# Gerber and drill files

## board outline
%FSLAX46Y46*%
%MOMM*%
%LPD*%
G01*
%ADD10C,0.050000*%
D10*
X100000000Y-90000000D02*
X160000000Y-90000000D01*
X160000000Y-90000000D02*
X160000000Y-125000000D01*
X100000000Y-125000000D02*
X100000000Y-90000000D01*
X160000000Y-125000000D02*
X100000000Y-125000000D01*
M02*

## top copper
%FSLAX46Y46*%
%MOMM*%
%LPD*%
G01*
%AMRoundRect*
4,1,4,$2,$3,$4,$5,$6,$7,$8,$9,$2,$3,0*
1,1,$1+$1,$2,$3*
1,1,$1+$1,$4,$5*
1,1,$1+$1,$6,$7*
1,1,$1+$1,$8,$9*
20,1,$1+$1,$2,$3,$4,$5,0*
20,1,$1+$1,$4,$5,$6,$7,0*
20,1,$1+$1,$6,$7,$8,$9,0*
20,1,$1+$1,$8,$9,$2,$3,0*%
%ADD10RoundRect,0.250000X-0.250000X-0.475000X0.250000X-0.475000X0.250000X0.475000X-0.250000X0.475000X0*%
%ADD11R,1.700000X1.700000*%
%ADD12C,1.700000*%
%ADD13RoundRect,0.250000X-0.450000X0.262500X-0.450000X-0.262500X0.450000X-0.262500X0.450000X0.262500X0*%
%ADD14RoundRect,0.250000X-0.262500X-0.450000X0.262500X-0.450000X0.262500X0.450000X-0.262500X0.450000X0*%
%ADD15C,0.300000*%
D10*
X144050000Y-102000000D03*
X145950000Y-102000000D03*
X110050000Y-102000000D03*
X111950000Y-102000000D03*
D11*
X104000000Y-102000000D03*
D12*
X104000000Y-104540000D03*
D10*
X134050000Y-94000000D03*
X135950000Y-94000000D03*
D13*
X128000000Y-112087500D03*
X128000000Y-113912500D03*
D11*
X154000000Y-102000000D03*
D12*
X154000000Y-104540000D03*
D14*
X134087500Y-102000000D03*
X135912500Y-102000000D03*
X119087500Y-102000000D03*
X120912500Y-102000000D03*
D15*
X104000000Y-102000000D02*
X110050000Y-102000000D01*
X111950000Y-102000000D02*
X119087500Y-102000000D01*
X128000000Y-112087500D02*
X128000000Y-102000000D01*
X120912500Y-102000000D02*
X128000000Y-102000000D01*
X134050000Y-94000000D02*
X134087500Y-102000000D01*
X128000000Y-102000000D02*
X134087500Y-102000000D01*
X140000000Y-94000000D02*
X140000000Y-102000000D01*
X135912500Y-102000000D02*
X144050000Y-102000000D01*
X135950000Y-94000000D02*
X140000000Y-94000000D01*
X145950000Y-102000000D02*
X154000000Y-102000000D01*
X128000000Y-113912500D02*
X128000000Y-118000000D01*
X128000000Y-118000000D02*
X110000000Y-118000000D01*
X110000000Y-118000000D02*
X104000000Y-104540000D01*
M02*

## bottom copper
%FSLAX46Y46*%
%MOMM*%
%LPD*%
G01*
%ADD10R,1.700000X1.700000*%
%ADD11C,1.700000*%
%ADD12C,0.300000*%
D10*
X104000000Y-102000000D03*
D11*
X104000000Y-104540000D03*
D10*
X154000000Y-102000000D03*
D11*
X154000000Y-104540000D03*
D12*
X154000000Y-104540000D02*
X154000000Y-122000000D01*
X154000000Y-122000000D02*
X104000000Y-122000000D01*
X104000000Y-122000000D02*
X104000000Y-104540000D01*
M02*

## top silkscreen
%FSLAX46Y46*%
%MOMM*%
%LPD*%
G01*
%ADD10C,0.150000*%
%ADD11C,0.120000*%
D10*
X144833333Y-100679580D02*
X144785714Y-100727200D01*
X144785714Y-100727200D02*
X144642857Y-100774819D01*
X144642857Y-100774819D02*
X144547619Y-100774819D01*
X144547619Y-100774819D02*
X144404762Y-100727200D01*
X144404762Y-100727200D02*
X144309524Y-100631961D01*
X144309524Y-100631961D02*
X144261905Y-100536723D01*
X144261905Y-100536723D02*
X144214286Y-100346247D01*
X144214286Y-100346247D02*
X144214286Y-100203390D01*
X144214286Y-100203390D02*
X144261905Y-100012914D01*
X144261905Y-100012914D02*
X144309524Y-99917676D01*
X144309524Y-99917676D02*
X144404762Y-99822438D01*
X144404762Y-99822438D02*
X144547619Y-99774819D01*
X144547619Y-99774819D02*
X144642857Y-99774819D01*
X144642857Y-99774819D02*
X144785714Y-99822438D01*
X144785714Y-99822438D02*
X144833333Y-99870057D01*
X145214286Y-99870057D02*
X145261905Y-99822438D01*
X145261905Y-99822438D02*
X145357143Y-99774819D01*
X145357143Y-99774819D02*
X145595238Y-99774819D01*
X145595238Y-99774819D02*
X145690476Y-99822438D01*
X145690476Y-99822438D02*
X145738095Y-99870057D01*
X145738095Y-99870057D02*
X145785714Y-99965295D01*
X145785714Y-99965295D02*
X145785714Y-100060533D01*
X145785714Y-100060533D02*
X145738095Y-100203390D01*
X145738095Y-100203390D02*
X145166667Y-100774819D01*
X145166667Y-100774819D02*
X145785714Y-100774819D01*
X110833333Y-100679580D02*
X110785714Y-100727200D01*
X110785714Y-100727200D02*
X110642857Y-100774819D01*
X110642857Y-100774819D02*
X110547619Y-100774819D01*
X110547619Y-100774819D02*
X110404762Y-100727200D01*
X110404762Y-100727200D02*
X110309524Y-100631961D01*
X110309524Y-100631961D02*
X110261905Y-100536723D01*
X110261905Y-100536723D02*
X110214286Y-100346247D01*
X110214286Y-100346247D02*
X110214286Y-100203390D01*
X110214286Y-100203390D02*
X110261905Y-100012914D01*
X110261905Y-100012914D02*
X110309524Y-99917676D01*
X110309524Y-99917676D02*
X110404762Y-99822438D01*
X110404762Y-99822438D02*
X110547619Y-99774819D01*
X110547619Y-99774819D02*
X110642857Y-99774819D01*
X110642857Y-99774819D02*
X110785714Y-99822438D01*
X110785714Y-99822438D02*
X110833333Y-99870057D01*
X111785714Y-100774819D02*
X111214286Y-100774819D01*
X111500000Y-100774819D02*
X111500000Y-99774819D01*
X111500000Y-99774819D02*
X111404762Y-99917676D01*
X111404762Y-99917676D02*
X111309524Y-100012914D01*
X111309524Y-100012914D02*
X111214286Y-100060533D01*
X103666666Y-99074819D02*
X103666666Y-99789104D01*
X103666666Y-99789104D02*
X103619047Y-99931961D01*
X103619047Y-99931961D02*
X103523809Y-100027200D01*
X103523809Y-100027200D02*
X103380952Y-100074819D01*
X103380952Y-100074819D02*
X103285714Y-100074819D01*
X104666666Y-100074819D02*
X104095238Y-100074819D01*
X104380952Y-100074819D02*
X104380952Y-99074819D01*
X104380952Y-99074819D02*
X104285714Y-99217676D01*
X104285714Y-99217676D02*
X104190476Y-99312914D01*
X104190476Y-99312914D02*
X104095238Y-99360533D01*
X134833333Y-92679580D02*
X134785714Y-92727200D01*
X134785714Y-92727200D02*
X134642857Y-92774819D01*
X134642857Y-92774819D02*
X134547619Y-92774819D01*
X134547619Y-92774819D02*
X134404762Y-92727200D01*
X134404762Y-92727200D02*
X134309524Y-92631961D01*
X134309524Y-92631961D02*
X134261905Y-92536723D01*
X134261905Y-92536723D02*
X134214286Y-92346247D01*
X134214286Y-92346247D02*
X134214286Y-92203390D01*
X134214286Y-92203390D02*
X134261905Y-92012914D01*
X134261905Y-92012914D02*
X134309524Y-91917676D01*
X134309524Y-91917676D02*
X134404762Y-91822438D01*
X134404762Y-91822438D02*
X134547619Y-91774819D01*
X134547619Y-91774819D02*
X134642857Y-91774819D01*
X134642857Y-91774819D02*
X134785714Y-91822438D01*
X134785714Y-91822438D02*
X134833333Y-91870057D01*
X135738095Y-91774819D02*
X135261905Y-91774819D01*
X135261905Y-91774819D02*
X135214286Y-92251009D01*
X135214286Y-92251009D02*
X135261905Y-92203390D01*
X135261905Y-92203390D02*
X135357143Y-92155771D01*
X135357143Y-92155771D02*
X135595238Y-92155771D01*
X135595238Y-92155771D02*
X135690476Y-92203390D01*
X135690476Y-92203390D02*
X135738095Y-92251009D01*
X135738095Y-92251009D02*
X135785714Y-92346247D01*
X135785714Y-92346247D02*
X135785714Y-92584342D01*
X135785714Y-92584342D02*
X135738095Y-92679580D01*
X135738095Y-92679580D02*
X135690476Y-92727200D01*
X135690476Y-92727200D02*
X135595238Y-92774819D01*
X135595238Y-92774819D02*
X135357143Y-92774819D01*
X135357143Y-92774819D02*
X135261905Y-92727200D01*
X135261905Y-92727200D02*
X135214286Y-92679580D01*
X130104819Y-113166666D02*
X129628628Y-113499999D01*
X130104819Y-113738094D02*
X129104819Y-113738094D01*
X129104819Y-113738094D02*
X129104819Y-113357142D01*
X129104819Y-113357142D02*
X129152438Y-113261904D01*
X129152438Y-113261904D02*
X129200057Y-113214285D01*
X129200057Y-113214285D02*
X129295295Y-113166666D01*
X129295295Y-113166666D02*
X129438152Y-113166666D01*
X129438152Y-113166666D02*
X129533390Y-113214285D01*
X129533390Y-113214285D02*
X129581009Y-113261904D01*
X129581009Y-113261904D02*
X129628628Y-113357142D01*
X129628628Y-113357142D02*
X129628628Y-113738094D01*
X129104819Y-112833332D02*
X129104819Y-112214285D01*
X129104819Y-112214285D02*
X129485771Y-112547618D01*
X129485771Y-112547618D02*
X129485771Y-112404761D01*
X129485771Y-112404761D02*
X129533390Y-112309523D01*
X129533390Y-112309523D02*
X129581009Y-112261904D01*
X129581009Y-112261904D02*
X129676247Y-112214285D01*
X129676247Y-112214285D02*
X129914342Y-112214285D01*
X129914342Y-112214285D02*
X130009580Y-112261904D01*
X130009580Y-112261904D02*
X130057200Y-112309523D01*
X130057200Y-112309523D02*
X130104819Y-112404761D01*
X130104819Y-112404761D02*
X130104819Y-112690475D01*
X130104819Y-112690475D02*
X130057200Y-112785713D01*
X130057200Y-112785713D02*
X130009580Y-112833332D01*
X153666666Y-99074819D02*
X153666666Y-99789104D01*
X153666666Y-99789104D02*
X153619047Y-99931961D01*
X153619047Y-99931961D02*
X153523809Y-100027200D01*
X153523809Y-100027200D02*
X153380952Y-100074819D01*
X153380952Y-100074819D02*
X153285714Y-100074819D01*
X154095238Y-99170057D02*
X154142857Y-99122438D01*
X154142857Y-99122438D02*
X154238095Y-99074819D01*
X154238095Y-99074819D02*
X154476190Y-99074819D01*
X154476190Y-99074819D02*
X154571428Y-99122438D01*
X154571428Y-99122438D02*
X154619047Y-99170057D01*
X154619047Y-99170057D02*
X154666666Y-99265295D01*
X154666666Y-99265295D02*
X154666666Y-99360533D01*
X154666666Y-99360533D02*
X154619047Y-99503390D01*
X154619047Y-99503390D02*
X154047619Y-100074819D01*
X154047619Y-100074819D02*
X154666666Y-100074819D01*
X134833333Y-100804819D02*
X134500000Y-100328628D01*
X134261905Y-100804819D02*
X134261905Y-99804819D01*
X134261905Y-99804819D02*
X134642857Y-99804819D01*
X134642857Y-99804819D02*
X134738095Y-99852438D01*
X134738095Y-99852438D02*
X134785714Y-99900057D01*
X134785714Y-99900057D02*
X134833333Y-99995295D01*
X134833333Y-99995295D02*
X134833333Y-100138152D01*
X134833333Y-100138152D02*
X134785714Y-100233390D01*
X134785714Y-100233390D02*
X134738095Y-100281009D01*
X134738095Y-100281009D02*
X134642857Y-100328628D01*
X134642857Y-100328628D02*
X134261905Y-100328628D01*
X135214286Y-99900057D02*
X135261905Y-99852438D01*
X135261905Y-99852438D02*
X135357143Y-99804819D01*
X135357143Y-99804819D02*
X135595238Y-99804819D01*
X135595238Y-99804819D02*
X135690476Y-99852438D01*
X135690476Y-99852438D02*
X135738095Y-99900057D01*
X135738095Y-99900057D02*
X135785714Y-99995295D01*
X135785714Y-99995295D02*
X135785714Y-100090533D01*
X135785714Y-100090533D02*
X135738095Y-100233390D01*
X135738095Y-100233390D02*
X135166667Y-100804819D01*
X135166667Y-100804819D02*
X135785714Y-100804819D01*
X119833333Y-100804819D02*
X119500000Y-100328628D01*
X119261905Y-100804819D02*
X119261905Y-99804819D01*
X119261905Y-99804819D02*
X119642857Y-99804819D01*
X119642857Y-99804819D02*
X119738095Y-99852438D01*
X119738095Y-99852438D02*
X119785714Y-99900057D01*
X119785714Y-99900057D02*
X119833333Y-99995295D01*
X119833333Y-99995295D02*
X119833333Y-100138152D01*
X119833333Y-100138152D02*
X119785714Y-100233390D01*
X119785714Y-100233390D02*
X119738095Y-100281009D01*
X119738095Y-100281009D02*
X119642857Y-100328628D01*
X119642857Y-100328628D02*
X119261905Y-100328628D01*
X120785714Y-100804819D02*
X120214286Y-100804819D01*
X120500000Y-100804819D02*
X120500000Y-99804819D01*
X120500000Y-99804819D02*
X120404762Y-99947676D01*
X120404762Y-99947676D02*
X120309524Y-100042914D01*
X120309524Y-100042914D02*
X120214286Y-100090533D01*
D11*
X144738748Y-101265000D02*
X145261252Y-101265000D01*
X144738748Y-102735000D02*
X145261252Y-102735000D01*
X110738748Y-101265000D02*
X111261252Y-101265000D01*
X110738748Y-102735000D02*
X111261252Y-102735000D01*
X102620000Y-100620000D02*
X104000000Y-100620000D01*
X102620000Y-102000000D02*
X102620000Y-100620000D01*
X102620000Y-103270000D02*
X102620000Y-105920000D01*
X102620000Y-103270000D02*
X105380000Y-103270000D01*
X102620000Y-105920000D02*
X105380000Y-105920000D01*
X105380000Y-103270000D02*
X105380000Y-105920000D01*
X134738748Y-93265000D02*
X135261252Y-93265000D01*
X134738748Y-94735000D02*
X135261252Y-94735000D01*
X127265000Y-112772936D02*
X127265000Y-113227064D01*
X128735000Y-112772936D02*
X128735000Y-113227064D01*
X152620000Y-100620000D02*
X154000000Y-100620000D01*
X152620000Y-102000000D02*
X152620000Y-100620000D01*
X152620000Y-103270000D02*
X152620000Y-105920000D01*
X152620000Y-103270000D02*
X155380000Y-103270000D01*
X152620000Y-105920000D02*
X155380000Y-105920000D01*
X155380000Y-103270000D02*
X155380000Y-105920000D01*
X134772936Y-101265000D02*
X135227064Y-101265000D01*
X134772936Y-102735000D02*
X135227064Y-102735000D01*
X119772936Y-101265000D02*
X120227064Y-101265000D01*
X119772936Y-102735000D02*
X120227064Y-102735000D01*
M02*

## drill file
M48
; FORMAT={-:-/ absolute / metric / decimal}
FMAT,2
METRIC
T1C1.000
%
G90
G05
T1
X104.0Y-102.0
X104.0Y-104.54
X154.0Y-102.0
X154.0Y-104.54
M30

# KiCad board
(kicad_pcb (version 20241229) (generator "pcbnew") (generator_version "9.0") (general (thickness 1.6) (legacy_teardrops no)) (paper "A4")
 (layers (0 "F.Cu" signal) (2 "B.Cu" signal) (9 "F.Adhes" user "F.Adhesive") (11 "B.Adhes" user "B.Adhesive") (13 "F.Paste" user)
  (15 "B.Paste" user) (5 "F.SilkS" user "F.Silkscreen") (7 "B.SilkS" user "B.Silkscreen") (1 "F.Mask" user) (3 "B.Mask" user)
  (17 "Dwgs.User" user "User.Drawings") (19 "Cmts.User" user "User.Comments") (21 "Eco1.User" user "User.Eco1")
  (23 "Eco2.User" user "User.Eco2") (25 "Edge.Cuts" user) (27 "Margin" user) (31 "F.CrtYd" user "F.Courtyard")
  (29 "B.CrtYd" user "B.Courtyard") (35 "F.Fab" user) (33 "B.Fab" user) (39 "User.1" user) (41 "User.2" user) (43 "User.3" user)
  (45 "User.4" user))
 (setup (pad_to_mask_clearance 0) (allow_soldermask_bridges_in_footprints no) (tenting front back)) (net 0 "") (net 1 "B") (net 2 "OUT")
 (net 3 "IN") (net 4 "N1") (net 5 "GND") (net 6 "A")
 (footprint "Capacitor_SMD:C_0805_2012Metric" (layer "F.Cu") (at 145 102)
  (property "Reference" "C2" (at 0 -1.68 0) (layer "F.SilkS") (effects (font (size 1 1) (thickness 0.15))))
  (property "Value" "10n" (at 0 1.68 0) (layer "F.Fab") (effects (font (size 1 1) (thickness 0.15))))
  (fp_line (start -0.261252 -0.735) (end 0.261252 -0.735) (stroke (width 0.12) (type solid)) (layer "F.SilkS"))
  (fp_line (start -0.261252 0.735) (end 0.261252 0.735) (stroke (width 0.12) (type solid)) (layer "F.SilkS"))
  (pad "1" smd roundrect (at -0.95 0) (size 1 1.45) (layers "F.Cu" "F.Mask" "F.Paste") (roundrect_rratio 0.25) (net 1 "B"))
  (pad "2" smd roundrect (at 0.95 0) (size 1 1.45) (layers "F.Cu" "F.Mask" "F.Paste") (roundrect_rratio 0.25) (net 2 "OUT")))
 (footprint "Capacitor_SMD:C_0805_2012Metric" (layer "F.Cu") (at 111 102)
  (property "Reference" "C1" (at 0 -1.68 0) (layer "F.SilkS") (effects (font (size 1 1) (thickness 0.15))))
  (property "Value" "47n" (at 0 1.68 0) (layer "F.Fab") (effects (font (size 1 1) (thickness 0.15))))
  (fp_line (start -0.261252 -0.735) (end 0.261252 -0.735) (stroke (width 0.12) (type solid)) (layer "F.SilkS"))
  (fp_line (start -0.261252 0.735) (end 0.261252 0.735) (stroke (width 0.12) (type solid)) (layer "F.SilkS"))
  (pad "1" smd roundrect (at -0.95 0) (size 1 1.45) (layers "F.Cu" "F.Mask" "F.Paste") (roundrect_rratio 0.25) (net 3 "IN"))
  (pad "2" smd roundrect (at 0.95 0) (size 1 1.45) (layers "F.Cu" "F.Mask" "F.Paste") (roundrect_rratio 0.25) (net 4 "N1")))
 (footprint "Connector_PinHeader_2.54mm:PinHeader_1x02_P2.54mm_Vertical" (layer "F.Cu") (at 104 102)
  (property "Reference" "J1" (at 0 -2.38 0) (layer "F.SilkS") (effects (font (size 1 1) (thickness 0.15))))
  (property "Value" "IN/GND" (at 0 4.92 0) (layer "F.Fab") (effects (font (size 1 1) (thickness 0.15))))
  (fp_line (start -1.38 -1.38) (end 0 -1.38) (stroke (width 0.12) (type solid)) (layer "F.SilkS"))
  (fp_line (start -1.38 0) (end -1.38 -1.38) (stroke (width 0.12) (type solid)) (layer "F.SilkS"))
  (fp_line (start -1.38 1.27) (end -1.38 3.92) (stroke (width 0.12) (type solid)) (layer "F.SilkS"))
  (fp_line (start -1.38 1.27) (end 1.38 1.27) (stroke (width 0.12) (type solid)) (layer "F.SilkS"))
  (fp_line (start -1.38 3.92) (end 1.38 3.92) (stroke (width 0.12) (type solid)) (layer "F.SilkS"))
  (fp_line (start 1.38 1.27) (end 1.38 3.92) (stroke (width 0.12) (type solid)) (layer "F.SilkS"))
  (pad "1" thru_hole rect (at 0 0) (size 1.7 1.7) (drill 1) (layers "*.Cu" "*.Mask") (remove_unused_layers no) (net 3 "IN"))
  (pad "2" thru_hole circle (at 0 2.54) (size 1.7 1.7) (drill 1) (layers "*.Cu" "*.Mask") (remove_unused_layers no) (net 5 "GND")))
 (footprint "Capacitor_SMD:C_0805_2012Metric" (layer "F.Cu") (at 135 94)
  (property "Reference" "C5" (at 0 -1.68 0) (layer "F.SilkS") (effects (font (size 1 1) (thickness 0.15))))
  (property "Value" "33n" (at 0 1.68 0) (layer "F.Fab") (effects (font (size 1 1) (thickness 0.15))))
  (fp_line (start -0.261252 -0.735) (end 0.261252 -0.735) (stroke (width 0.12) (type solid)) (layer "F.SilkS"))
  (fp_line (start -0.261252 0.735) (end 0.261252 0.735) (stroke (width 0.12) (type solid)) (layer "F.SilkS"))
  (pad "1" smd roundrect (at -0.95 0) (size 1 1.45) (layers "F.Cu" "F.Mask" "F.Paste") (roundrect_rratio 0.25) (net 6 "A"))
  (pad "2" smd roundrect (at 0.95 0) (size 1 1.45) (layers "F.Cu" "F.Mask" "F.Paste") (roundrect_rratio 0.25) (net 1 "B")))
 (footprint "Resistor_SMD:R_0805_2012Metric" (layer "F.Cu") (at 128 113 -90)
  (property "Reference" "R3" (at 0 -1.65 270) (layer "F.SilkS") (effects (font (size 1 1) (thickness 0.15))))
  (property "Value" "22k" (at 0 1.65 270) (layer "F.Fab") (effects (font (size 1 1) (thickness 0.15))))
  (fp_line (start -0.227064 0.735) (end 0.227064 0.735) (stroke (width 0.12) (type solid)) (layer "F.SilkS"))
  (fp_line (start -0.227064 -0.735) (end 0.227064 -0.735) (stroke (width 0.12) (type solid)) (layer "F.SilkS"))
  (pad "1" smd roundrect (at -0.9125 0 270) (size 1.025 1.4) (layers "F.Cu" "F.Mask" "F.Paste") (roundrect_rratio 0.243902) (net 6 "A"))
  (pad "2" smd roundrect (at 0.9125 0 270) (size 1.025 1.4) (layers "F.Cu" "F.Mask" "F.Paste") (roundrect_rratio 0.243902) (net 5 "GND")))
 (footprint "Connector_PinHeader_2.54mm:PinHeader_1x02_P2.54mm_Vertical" (layer "F.Cu") (at 154 102)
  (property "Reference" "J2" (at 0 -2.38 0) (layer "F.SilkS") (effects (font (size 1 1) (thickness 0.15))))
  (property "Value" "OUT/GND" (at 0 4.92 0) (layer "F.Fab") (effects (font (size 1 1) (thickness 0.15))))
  (fp_line (start -1.38 -1.38) (end 0 -1.38) (stroke (width 0.12) (type solid)) (layer "F.SilkS"))
  (fp_line (start -1.38 0) (end -1.38 -1.38) (stroke (width 0.12) (type solid)) (layer "F.SilkS"))
  (fp_line (start -1.38 1.27) (end -1.38 3.92) (stroke (width 0.12) (type solid)) (layer "F.SilkS"))
  (fp_line (start -1.38 1.27) (end 1.38 1.27) (stroke (width 0.12) (type solid)) (layer "F.SilkS"))
  (fp_line (start -1.38 3.92) (end 1.38 3.92) (stroke (width 0.12) (type solid)) (layer "F.SilkS"))
  (fp_line (start 1.38 1.27) (end 1.38 3.92) (stroke (width 0.12) (type solid)) (layer "F.SilkS"))
  (pad "1" thru_hole rect (at 0 0) (size 1.7 1.7) (drill 1) (layers "*.Cu" "*.Mask") (remove_unused_layers no) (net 2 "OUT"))
  (pad "2" thru_hole circle (at 0 2.54) (size 1.7 1.7) (drill 1) (layers "*.Cu" "*.Mask") (remove_unused_layers no) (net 5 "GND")))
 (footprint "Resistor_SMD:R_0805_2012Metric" (layer "F.Cu") (at 135 102)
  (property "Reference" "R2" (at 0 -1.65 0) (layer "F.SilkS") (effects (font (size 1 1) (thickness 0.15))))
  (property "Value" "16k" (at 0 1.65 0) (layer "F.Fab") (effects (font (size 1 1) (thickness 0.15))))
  (fp_line (start -0.227064 -0.735) (end 0.227064 -0.735) (stroke (width 0.12) (type solid)) (layer "F.SilkS"))
  (fp_line (start -0.227064 0.735) (end 0.227064 0.735) (stroke (width 0.12) (type solid)) (layer "F.SilkS"))
  (pad "1" smd roundrect (at -0.9125 0) (size 1.025 1.4) (layers "F.Cu" "F.Mask" "F.Paste") (roundrect_rratio 0.243902) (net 6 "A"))
  (pad "2" smd roundrect (at 0.9125 0) (size 1.025 1.4) (layers "F.Cu" "F.Mask" "F.Paste") (roundrect_rratio 0.243902) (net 1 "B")))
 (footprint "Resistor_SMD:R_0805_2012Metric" (layer "F.Cu") (at 120 102)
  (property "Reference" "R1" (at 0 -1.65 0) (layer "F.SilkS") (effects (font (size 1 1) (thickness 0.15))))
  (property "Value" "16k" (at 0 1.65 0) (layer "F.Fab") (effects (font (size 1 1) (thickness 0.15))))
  (fp_line (start -0.227064 -0.735) (end 0.227064 -0.735) (stroke (width 0.12) (type solid)) (layer "F.SilkS"))
  (fp_line (start -0.227064 0.735) (end 0.227064 0.735) (stroke (width 0.12) (type solid)) (layer "F.SilkS"))
  (pad "1" smd roundrect (at -0.9125 0) (size 1.025 1.4) (layers "F.Cu" "F.Mask" "F.Paste") (roundrect_rratio 0.243902) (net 4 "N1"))
  (pad "2" smd roundrect (at 0.9125 0) (size 1.025 1.4) (layers "F.Cu" "F.Mask" "F.Paste") (roundrect_rratio 0.243902) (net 6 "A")))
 (gr_line (start 100 90) (end 160 90) (stroke (width 0.05) (type default)) (layer "Edge.Cuts"))
 (gr_line (start 160 90) (end 160 125) (stroke (width 0.05) (type default)) (layer "Edge.Cuts"))
 (gr_line (start 100 125) (end 100 90) (stroke (width 0.05) (type default)) (layer "Edge.Cuts"))
 (gr_line (start 160 125) (end 100 125) (stroke (width 0.05) (type default)) (layer "Edge.Cuts"))
 (segment (start 104 102) (end 110.05 102) (width 0.3) (layer "F.Cu") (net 3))
 (segment (start 111.95 102) (end 119.0875 102) (width 0.3) (layer "F.Cu") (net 4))
 (segment (start 128 112.0875) (end 128 102) (width 0.3) (layer "F.Cu") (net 6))
 (segment (start 120.9125 102) (end 128 102) (width 0.3) (layer "F.Cu") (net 6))
 (segment (start 134.05 94) (end 134.0875 102) (width 0.3) (layer "F.Cu") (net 6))
 (segment (start 128 102) (end 134.0875 102) (width 0.3) (layer "F.Cu") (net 6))
 (segment (start 140 94) (end 140 102) (width 0.3) (layer "F.Cu") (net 1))
 (segment (start 135.9125 102) (end 144.05 102) (width 0.3) (layer "F.Cu") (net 1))
 (segment (start 135.95 94) (end 140 94) (width 0.3) (layer "F.Cu") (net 1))
 (segment (start 145.95 102) (end 154 102) (width 0.3) (layer "F.Cu") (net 2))
 (segment (start 128 113.9125) (end 128 118) (width 0.3) (layer "F.Cu") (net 5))
 (segment (start 128 118) (end 110 118) (width 0.3) (layer "F.Cu") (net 5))
 (segment (start 110 118) (end 104 104.54) (width 0.3) (layer "F.Cu") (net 5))
 (segment (start 154 104.54) (end 154 122) (width 0.3) (layer "B.Cu") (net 5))
 (segment (start 154 122) (end 104 122) (width 0.3) (layer "B.Cu") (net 5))
 (segment (start 104 122) (end 104 104.54) (width 0.3) (layer "B.Cu") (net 5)))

